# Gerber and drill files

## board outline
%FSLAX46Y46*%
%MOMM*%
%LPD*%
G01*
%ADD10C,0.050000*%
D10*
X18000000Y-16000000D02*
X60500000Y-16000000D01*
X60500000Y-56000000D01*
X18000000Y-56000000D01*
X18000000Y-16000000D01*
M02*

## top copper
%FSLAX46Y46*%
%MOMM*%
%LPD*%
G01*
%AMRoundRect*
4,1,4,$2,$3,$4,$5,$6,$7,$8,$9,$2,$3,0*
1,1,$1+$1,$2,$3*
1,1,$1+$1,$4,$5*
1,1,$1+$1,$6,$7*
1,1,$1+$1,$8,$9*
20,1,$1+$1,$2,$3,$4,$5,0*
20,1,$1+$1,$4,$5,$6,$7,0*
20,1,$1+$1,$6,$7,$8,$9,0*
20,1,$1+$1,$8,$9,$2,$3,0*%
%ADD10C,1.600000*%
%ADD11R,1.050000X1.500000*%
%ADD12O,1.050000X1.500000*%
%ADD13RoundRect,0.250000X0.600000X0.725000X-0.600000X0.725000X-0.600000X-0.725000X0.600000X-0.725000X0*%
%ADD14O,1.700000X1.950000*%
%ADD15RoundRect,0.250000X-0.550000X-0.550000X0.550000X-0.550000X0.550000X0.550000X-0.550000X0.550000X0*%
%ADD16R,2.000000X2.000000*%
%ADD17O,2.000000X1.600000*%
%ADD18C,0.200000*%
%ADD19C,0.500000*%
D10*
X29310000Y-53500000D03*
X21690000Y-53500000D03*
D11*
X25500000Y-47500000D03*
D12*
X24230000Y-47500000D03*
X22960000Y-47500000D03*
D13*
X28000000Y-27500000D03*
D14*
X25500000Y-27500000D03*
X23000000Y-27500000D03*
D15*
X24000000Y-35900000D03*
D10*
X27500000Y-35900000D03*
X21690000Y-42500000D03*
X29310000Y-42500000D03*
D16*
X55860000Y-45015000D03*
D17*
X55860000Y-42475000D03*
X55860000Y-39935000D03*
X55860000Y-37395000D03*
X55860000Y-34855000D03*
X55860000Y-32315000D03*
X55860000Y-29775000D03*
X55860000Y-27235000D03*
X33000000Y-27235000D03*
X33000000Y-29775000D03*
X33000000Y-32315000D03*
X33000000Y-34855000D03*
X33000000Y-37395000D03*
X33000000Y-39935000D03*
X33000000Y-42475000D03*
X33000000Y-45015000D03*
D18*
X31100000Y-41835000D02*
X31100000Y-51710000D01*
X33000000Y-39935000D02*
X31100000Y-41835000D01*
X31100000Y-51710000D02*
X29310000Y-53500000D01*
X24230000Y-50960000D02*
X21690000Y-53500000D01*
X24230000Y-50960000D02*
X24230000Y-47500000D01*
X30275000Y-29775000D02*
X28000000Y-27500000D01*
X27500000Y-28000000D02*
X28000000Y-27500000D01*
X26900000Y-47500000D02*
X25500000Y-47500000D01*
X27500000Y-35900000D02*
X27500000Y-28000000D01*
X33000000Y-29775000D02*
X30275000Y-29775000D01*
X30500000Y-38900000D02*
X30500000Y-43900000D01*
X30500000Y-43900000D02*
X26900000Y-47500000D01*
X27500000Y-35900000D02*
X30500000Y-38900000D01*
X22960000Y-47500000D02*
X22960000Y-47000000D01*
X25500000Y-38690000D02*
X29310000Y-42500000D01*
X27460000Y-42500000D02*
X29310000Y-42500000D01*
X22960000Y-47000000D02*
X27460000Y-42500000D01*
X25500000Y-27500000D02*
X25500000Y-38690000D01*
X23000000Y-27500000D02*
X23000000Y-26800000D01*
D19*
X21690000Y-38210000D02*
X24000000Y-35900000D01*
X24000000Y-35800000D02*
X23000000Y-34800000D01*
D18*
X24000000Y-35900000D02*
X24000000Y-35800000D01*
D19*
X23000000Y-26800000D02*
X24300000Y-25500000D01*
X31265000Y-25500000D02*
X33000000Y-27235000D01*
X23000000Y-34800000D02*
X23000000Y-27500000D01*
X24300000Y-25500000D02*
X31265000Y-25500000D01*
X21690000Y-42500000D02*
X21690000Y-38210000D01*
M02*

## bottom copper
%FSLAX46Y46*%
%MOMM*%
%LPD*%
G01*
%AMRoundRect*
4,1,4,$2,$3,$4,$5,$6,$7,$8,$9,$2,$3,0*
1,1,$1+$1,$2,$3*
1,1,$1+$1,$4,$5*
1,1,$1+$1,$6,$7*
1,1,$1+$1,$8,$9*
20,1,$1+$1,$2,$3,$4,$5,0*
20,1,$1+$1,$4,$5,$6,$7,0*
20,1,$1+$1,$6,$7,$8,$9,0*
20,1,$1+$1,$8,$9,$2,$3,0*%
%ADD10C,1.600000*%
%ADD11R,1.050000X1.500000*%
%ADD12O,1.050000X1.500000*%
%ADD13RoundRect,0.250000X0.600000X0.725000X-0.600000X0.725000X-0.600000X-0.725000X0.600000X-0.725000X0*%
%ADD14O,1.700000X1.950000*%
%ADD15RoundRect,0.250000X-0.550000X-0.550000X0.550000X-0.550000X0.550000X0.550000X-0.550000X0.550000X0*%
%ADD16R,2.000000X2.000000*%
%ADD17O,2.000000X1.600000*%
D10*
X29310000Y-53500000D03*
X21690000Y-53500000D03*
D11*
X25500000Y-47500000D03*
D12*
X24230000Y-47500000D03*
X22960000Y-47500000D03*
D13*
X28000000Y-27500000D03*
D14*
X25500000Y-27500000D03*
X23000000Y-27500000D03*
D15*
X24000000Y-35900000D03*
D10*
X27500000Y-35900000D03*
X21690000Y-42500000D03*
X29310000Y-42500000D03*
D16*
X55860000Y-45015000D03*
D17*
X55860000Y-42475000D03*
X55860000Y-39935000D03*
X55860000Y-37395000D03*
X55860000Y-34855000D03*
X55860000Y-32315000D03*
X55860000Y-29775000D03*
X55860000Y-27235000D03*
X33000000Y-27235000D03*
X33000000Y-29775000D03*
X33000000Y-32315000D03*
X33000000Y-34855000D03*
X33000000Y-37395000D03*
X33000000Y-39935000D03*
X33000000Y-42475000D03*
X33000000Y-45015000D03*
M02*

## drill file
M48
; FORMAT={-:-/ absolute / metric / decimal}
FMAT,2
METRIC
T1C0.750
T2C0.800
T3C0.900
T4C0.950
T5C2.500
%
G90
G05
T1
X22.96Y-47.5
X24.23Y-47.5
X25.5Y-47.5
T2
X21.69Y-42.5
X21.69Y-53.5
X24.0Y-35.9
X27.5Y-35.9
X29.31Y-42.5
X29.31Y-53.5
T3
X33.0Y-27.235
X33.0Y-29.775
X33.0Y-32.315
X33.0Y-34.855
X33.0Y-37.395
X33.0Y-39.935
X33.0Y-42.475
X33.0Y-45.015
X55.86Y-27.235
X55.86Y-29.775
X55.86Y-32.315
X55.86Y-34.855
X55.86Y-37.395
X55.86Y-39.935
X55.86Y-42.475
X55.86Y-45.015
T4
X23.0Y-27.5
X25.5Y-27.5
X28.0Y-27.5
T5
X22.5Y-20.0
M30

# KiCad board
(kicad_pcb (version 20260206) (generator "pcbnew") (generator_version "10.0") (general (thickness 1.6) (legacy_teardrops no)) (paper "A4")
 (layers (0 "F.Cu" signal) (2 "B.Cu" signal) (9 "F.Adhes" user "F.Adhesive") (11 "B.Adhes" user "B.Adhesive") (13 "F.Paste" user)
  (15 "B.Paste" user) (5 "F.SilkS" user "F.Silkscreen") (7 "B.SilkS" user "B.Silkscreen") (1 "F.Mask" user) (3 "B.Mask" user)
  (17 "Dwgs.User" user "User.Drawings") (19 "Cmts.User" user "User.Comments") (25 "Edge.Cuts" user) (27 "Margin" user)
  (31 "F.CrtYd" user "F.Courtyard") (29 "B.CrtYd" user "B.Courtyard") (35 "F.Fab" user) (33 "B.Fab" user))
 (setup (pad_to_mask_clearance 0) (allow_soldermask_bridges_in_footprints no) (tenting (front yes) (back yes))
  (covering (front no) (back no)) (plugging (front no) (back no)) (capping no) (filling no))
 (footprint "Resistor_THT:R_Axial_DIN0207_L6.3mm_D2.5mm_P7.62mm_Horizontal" (layer "F.Cu") (at 29.31 53.5 180)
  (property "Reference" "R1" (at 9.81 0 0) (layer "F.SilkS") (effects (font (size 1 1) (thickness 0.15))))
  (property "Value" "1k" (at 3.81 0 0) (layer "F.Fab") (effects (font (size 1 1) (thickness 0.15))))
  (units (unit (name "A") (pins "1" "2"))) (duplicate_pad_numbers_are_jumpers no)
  (pad "1" thru_hole circle (at 0 0 180) (size 1.6 1.6) (drill 0.8) (layers "*.Cu" "*.Mask") (remove_unused_layers no) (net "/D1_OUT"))
  (pad "2" thru_hole circle (at 7.62 0 180) (size 1.6 1.6) (drill 0.8) (layers "*.Cu" "*.Mask") (remove_unused_layers no) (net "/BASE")))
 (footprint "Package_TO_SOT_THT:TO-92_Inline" (layer "F.Cu") (at 25.5 47.5 180)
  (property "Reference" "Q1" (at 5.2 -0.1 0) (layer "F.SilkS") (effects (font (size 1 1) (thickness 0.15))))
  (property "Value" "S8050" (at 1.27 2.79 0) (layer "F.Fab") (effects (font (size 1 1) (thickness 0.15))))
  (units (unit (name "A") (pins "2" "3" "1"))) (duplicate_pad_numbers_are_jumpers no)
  (pad "1" thru_hole rect (at 0 0 180) (size 1.05 1.5) (drill 0.75) (layers "*.Cu" "*.Mask") (remove_unused_layers no) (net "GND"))
  (pad "2" thru_hole oval (at 1.27 0 180) (size 1.05 1.5) (drill 0.75) (layers "*.Cu" "*.Mask") (remove_unused_layers no) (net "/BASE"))
  (pad "3" thru_hole oval (at 2.54 0 180) (size 1.05 1.5) (drill 0.75) (layers "*.Cu" "*.Mask") (remove_unused_layers no) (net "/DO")))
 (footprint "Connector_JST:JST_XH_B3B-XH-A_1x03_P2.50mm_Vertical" (layer "F.Cu") (at 28 27.5 180)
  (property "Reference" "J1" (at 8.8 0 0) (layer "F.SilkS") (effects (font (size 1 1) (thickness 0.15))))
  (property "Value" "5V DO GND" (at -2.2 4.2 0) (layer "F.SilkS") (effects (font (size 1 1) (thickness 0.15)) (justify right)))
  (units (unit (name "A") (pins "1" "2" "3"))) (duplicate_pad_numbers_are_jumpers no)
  (pad "1" thru_hole roundrect (at 0 0 180) (size 1.7 1.95) (drill 0.95) (layers "*.Cu" "*.Mask") (remove_unused_layers no)
   (roundrect_rratio 0.147059) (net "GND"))
  (pad "2" thru_hole oval (at 2.5 0 180) (size 1.7 1.95) (drill 0.95) (layers "*.Cu" "*.Mask") (remove_unused_layers no) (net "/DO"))
  (pad "3" thru_hole oval (at 5 0 180) (size 1.7 1.95) (drill 0.95) (layers "*.Cu" "*.Mask") (remove_unused_layers no) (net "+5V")))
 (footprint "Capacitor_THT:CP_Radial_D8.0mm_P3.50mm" (layer "F.Cu") (at 24 35.9)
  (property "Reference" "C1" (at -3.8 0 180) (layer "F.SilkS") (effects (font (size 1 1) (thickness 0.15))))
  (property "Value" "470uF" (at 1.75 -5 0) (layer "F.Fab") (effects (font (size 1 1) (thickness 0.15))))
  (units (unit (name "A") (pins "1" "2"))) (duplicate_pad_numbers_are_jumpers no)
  (pad "1" thru_hole roundrect (at 0 0) (size 1.6 1.6) (drill 0.8) (layers "*.Cu" "*.Mask") (remove_unused_layers no)
   (roundrect_rratio 0.15625) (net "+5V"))
  (pad "2" thru_hole circle (at 3.5 0) (size 1.6 1.6) (drill 0.8) (layers "*.Cu" "*.Mask") (remove_unused_layers no) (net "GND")))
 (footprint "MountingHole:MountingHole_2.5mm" (layer "F.Cu") (at 22.5 20)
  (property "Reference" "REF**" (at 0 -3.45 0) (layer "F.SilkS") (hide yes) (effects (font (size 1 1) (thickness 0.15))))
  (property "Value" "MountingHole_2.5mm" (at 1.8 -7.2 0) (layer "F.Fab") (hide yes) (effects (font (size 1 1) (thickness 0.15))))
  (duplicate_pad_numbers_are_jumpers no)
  (pad "" np_thru_hole circle (at 0 0) (size 2.5 2.5) (drill 2.5) (layers "*.Cu" "*.Mask")))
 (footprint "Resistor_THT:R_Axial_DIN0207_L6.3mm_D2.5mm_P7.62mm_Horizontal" (layer "F.Cu") (at 21.69 42.5)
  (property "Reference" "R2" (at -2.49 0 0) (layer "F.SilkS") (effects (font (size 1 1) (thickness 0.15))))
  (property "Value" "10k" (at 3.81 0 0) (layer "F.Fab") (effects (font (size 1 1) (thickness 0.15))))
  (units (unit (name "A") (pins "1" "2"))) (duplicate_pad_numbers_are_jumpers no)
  (pad "1" thru_hole circle (at 0 0) (size 1.6 1.6) (drill 0.8) (layers "*.Cu" "*.Mask") (remove_unused_layers no) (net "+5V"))
  (pad "2" thru_hole circle (at 7.62 0) (size 1.6 1.6) (drill 0.8) (layers "*.Cu" "*.Mask") (remove_unused_layers no) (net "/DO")))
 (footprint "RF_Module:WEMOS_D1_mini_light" (layer "F.Cu") (at 55.86 45.015 180)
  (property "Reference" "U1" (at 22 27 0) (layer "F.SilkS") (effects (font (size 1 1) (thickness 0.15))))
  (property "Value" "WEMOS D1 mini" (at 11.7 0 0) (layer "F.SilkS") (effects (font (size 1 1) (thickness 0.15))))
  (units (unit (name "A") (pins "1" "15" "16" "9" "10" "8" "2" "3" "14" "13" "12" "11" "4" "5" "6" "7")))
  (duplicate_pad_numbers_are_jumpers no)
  (pad "1" thru_hole rect (at 0 0 180) (size 2 2) (drill 0.9) (layers "*.Cu" "*.Mask") (remove_unused_layers no)
   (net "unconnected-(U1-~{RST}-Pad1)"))
  (pad "2" thru_hole oval (at 0 2.54 180) (size 2 1.6) (drill 0.9) (layers "*.Cu" "*.Mask") (remove_unused_layers no)
   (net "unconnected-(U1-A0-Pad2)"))
  (pad "3" thru_hole oval (at 0 5.08 180) (size 2 1.6) (drill 0.9) (layers "*.Cu" "*.Mask") (remove_unused_layers no)
   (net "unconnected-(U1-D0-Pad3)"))
  (pad "4" thru_hole oval (at 0 7.62 180) (size 2 1.6) (drill 0.9) (layers "*.Cu" "*.Mask") (remove_unused_layers no)
   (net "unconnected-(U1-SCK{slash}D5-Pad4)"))
  (pad "5" thru_hole oval (at 0 10.16 180) (size 2 1.6) (drill 0.9) (layers "*.Cu" "*.Mask") (remove_unused_layers no)
   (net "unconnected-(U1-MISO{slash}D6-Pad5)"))
  (pad "6" thru_hole oval (at 0 12.7 180) (size 2 1.6) (drill 0.9) (layers "*.Cu" "*.Mask") (remove_unused_layers no)
   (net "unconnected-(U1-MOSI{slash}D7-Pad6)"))
  (pad "7" thru_hole oval (at 0 15.24 180) (size 2 1.6) (drill 0.9) (layers "*.Cu" "*.Mask") (remove_unused_layers no)
   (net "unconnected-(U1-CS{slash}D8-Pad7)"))
  (pad "8" thru_hole oval (at 0 17.78 180) (size 2 1.6) (drill 0.9) (layers "*.Cu" "*.Mask") (remove_unused_layers no)
   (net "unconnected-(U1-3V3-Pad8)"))
  (pad "9" thru_hole oval (at 22.86 17.78 180) (size 2 1.6) (drill 0.9) (layers "*.Cu" "*.Mask") (remove_unused_layers no) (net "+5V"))
  (pad "10" thru_hole oval (at 22.86 15.24 180) (size 2 1.6) (drill 0.9) (layers "*.Cu" "*.Mask") (remove_unused_layers no) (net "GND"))
  (pad "11" thru_hole oval (at 22.86 12.7 180) (size 2 1.6) (drill 0.9) (layers "*.Cu" "*.Mask") (remove_unused_layers no)
   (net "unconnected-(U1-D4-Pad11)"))
  (pad "12" thru_hole oval (at 22.86 10.16 180) (size 2 1.6) (drill 0.9) (layers "*.Cu" "*.Mask") (remove_unused_layers no)
   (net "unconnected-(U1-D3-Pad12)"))
  (pad "13" thru_hole oval (at 22.86 7.62 180) (size 2 1.6) (drill 0.9) (layers "*.Cu" "*.Mask") (remove_unused_layers no)
   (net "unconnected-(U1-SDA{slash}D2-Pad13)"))
  (pad "14" thru_hole oval (at 22.86 5.08 180) (size 2 1.6) (drill 0.9) (layers "*.Cu" "*.Mask") (remove_unused_layers no) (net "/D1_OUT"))
  (pad "15" thru_hole oval (at 22.86 2.54 180) (size 2 1.6) (drill 0.9) (layers "*.Cu" "*.Mask") (remove_unused_layers no)
   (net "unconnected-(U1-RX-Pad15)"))
  (pad "16" thru_hole oval (at 22.86 0 180) (size 2 1.6) (drill 0.9) (layers "*.Cu" "*.Mask") (remove_unused_layers no)
   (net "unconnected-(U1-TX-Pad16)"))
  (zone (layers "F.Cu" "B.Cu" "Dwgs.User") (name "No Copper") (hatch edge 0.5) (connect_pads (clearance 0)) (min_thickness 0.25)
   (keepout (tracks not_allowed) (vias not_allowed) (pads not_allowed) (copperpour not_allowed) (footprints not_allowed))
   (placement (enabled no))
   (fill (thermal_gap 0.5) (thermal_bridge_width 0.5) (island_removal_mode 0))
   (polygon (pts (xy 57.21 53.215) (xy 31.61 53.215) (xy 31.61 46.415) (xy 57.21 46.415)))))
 (gr_rect (start 18 16) (end 60.5 56) (stroke (width 0.05) (type default)) (fill no) (layer "Edge.Cuts"))
 (segment (start 31.1 41.835) (end 31.1 51.71) (width 0.2) (layer "F.Cu") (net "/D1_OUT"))
 (segment (start 33 39.935) (end 31.1 41.835) (width 0.2) (layer "F.Cu") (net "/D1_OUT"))
 (segment (start 31.1 51.71) (end 29.31 53.5) (width 0.2) (layer "F.Cu") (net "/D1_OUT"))
 (segment (start 24.23 50.96) (end 21.69 53.5) (width 0.2) (layer "F.Cu") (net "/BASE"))
 (segment (start 24.23 50.96) (end 24.23 47.5) (width 0.2) (layer "F.Cu") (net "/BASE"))
 (segment (start 30.275 29.775) (end 28 27.5) (width 0.2) (layer "F.Cu") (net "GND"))
 (segment (start 27.5 28) (end 28 27.5) (width 0.2) (layer "F.Cu") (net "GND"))
 (segment (start 26.9 47.5) (end 25.5 47.5) (width 0.2) (layer "F.Cu") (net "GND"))
 (segment (start 27.5 35.9) (end 27.5 28) (width 0.2) (layer "F.Cu") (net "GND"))
 (segment (start 33 29.775) (end 30.275 29.775) (width 0.2) (layer "F.Cu") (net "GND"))
 (segment (start 30.5 38.9) (end 30.5 43.9) (width 0.2) (layer "F.Cu") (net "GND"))
 (segment (start 30.5 43.9) (end 26.9 47.5) (width 0.2) (layer "F.Cu") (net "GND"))
 (segment (start 27.5 35.9) (end 30.5 38.9) (width 0.2) (layer "F.Cu") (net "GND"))
 (segment (start 22.96 47.5) (end 22.96 47) (width 0.2) (layer "F.Cu") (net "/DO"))
 (segment (start 25.5 38.69) (end 29.31 42.5) (width 0.2) (layer "F.Cu") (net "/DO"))
 (segment (start 27.46 42.5) (end 29.31 42.5) (width 0.2) (layer "F.Cu") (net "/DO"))
 (segment (start 22.96 47) (end 27.46 42.5) (width 0.2) (layer "F.Cu") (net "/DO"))
 (segment (start 25.5 27.5) (end 25.5 38.69) (width 0.2) (layer "F.Cu") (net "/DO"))
 (segment (start 23 27.5) (end 23 26.8) (width 0.2) (layer "F.Cu") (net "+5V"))
 (segment (start 21.69 38.21) (end 24 35.9) (width 0.5) (layer "F.Cu") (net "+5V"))
 (segment (start 24 35.8) (end 23 34.8) (width 0.5) (layer "F.Cu") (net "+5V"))
 (segment (start 24 35.9) (end 24 35.8) (width 0.2) (layer "F.Cu") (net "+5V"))
 (segment (start 23 26.8) (end 24.3 25.5) (width 0.5) (layer "F.Cu") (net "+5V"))
 (segment (start 31.265 25.5) (end 33 27.235) (width 0.5) (layer "F.Cu") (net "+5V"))
 (segment (start 23 34.8) (end 23 27.5) (width 0.5) (layer "F.Cu") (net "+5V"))
 (segment (start 24.3 25.5) (end 31.265 25.5) (width 0.5) (layer "F.Cu") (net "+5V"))
 (segment (start 21.69 42.5) (end 21.69 38.21) (width 0.5) (layer "F.Cu") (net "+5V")))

